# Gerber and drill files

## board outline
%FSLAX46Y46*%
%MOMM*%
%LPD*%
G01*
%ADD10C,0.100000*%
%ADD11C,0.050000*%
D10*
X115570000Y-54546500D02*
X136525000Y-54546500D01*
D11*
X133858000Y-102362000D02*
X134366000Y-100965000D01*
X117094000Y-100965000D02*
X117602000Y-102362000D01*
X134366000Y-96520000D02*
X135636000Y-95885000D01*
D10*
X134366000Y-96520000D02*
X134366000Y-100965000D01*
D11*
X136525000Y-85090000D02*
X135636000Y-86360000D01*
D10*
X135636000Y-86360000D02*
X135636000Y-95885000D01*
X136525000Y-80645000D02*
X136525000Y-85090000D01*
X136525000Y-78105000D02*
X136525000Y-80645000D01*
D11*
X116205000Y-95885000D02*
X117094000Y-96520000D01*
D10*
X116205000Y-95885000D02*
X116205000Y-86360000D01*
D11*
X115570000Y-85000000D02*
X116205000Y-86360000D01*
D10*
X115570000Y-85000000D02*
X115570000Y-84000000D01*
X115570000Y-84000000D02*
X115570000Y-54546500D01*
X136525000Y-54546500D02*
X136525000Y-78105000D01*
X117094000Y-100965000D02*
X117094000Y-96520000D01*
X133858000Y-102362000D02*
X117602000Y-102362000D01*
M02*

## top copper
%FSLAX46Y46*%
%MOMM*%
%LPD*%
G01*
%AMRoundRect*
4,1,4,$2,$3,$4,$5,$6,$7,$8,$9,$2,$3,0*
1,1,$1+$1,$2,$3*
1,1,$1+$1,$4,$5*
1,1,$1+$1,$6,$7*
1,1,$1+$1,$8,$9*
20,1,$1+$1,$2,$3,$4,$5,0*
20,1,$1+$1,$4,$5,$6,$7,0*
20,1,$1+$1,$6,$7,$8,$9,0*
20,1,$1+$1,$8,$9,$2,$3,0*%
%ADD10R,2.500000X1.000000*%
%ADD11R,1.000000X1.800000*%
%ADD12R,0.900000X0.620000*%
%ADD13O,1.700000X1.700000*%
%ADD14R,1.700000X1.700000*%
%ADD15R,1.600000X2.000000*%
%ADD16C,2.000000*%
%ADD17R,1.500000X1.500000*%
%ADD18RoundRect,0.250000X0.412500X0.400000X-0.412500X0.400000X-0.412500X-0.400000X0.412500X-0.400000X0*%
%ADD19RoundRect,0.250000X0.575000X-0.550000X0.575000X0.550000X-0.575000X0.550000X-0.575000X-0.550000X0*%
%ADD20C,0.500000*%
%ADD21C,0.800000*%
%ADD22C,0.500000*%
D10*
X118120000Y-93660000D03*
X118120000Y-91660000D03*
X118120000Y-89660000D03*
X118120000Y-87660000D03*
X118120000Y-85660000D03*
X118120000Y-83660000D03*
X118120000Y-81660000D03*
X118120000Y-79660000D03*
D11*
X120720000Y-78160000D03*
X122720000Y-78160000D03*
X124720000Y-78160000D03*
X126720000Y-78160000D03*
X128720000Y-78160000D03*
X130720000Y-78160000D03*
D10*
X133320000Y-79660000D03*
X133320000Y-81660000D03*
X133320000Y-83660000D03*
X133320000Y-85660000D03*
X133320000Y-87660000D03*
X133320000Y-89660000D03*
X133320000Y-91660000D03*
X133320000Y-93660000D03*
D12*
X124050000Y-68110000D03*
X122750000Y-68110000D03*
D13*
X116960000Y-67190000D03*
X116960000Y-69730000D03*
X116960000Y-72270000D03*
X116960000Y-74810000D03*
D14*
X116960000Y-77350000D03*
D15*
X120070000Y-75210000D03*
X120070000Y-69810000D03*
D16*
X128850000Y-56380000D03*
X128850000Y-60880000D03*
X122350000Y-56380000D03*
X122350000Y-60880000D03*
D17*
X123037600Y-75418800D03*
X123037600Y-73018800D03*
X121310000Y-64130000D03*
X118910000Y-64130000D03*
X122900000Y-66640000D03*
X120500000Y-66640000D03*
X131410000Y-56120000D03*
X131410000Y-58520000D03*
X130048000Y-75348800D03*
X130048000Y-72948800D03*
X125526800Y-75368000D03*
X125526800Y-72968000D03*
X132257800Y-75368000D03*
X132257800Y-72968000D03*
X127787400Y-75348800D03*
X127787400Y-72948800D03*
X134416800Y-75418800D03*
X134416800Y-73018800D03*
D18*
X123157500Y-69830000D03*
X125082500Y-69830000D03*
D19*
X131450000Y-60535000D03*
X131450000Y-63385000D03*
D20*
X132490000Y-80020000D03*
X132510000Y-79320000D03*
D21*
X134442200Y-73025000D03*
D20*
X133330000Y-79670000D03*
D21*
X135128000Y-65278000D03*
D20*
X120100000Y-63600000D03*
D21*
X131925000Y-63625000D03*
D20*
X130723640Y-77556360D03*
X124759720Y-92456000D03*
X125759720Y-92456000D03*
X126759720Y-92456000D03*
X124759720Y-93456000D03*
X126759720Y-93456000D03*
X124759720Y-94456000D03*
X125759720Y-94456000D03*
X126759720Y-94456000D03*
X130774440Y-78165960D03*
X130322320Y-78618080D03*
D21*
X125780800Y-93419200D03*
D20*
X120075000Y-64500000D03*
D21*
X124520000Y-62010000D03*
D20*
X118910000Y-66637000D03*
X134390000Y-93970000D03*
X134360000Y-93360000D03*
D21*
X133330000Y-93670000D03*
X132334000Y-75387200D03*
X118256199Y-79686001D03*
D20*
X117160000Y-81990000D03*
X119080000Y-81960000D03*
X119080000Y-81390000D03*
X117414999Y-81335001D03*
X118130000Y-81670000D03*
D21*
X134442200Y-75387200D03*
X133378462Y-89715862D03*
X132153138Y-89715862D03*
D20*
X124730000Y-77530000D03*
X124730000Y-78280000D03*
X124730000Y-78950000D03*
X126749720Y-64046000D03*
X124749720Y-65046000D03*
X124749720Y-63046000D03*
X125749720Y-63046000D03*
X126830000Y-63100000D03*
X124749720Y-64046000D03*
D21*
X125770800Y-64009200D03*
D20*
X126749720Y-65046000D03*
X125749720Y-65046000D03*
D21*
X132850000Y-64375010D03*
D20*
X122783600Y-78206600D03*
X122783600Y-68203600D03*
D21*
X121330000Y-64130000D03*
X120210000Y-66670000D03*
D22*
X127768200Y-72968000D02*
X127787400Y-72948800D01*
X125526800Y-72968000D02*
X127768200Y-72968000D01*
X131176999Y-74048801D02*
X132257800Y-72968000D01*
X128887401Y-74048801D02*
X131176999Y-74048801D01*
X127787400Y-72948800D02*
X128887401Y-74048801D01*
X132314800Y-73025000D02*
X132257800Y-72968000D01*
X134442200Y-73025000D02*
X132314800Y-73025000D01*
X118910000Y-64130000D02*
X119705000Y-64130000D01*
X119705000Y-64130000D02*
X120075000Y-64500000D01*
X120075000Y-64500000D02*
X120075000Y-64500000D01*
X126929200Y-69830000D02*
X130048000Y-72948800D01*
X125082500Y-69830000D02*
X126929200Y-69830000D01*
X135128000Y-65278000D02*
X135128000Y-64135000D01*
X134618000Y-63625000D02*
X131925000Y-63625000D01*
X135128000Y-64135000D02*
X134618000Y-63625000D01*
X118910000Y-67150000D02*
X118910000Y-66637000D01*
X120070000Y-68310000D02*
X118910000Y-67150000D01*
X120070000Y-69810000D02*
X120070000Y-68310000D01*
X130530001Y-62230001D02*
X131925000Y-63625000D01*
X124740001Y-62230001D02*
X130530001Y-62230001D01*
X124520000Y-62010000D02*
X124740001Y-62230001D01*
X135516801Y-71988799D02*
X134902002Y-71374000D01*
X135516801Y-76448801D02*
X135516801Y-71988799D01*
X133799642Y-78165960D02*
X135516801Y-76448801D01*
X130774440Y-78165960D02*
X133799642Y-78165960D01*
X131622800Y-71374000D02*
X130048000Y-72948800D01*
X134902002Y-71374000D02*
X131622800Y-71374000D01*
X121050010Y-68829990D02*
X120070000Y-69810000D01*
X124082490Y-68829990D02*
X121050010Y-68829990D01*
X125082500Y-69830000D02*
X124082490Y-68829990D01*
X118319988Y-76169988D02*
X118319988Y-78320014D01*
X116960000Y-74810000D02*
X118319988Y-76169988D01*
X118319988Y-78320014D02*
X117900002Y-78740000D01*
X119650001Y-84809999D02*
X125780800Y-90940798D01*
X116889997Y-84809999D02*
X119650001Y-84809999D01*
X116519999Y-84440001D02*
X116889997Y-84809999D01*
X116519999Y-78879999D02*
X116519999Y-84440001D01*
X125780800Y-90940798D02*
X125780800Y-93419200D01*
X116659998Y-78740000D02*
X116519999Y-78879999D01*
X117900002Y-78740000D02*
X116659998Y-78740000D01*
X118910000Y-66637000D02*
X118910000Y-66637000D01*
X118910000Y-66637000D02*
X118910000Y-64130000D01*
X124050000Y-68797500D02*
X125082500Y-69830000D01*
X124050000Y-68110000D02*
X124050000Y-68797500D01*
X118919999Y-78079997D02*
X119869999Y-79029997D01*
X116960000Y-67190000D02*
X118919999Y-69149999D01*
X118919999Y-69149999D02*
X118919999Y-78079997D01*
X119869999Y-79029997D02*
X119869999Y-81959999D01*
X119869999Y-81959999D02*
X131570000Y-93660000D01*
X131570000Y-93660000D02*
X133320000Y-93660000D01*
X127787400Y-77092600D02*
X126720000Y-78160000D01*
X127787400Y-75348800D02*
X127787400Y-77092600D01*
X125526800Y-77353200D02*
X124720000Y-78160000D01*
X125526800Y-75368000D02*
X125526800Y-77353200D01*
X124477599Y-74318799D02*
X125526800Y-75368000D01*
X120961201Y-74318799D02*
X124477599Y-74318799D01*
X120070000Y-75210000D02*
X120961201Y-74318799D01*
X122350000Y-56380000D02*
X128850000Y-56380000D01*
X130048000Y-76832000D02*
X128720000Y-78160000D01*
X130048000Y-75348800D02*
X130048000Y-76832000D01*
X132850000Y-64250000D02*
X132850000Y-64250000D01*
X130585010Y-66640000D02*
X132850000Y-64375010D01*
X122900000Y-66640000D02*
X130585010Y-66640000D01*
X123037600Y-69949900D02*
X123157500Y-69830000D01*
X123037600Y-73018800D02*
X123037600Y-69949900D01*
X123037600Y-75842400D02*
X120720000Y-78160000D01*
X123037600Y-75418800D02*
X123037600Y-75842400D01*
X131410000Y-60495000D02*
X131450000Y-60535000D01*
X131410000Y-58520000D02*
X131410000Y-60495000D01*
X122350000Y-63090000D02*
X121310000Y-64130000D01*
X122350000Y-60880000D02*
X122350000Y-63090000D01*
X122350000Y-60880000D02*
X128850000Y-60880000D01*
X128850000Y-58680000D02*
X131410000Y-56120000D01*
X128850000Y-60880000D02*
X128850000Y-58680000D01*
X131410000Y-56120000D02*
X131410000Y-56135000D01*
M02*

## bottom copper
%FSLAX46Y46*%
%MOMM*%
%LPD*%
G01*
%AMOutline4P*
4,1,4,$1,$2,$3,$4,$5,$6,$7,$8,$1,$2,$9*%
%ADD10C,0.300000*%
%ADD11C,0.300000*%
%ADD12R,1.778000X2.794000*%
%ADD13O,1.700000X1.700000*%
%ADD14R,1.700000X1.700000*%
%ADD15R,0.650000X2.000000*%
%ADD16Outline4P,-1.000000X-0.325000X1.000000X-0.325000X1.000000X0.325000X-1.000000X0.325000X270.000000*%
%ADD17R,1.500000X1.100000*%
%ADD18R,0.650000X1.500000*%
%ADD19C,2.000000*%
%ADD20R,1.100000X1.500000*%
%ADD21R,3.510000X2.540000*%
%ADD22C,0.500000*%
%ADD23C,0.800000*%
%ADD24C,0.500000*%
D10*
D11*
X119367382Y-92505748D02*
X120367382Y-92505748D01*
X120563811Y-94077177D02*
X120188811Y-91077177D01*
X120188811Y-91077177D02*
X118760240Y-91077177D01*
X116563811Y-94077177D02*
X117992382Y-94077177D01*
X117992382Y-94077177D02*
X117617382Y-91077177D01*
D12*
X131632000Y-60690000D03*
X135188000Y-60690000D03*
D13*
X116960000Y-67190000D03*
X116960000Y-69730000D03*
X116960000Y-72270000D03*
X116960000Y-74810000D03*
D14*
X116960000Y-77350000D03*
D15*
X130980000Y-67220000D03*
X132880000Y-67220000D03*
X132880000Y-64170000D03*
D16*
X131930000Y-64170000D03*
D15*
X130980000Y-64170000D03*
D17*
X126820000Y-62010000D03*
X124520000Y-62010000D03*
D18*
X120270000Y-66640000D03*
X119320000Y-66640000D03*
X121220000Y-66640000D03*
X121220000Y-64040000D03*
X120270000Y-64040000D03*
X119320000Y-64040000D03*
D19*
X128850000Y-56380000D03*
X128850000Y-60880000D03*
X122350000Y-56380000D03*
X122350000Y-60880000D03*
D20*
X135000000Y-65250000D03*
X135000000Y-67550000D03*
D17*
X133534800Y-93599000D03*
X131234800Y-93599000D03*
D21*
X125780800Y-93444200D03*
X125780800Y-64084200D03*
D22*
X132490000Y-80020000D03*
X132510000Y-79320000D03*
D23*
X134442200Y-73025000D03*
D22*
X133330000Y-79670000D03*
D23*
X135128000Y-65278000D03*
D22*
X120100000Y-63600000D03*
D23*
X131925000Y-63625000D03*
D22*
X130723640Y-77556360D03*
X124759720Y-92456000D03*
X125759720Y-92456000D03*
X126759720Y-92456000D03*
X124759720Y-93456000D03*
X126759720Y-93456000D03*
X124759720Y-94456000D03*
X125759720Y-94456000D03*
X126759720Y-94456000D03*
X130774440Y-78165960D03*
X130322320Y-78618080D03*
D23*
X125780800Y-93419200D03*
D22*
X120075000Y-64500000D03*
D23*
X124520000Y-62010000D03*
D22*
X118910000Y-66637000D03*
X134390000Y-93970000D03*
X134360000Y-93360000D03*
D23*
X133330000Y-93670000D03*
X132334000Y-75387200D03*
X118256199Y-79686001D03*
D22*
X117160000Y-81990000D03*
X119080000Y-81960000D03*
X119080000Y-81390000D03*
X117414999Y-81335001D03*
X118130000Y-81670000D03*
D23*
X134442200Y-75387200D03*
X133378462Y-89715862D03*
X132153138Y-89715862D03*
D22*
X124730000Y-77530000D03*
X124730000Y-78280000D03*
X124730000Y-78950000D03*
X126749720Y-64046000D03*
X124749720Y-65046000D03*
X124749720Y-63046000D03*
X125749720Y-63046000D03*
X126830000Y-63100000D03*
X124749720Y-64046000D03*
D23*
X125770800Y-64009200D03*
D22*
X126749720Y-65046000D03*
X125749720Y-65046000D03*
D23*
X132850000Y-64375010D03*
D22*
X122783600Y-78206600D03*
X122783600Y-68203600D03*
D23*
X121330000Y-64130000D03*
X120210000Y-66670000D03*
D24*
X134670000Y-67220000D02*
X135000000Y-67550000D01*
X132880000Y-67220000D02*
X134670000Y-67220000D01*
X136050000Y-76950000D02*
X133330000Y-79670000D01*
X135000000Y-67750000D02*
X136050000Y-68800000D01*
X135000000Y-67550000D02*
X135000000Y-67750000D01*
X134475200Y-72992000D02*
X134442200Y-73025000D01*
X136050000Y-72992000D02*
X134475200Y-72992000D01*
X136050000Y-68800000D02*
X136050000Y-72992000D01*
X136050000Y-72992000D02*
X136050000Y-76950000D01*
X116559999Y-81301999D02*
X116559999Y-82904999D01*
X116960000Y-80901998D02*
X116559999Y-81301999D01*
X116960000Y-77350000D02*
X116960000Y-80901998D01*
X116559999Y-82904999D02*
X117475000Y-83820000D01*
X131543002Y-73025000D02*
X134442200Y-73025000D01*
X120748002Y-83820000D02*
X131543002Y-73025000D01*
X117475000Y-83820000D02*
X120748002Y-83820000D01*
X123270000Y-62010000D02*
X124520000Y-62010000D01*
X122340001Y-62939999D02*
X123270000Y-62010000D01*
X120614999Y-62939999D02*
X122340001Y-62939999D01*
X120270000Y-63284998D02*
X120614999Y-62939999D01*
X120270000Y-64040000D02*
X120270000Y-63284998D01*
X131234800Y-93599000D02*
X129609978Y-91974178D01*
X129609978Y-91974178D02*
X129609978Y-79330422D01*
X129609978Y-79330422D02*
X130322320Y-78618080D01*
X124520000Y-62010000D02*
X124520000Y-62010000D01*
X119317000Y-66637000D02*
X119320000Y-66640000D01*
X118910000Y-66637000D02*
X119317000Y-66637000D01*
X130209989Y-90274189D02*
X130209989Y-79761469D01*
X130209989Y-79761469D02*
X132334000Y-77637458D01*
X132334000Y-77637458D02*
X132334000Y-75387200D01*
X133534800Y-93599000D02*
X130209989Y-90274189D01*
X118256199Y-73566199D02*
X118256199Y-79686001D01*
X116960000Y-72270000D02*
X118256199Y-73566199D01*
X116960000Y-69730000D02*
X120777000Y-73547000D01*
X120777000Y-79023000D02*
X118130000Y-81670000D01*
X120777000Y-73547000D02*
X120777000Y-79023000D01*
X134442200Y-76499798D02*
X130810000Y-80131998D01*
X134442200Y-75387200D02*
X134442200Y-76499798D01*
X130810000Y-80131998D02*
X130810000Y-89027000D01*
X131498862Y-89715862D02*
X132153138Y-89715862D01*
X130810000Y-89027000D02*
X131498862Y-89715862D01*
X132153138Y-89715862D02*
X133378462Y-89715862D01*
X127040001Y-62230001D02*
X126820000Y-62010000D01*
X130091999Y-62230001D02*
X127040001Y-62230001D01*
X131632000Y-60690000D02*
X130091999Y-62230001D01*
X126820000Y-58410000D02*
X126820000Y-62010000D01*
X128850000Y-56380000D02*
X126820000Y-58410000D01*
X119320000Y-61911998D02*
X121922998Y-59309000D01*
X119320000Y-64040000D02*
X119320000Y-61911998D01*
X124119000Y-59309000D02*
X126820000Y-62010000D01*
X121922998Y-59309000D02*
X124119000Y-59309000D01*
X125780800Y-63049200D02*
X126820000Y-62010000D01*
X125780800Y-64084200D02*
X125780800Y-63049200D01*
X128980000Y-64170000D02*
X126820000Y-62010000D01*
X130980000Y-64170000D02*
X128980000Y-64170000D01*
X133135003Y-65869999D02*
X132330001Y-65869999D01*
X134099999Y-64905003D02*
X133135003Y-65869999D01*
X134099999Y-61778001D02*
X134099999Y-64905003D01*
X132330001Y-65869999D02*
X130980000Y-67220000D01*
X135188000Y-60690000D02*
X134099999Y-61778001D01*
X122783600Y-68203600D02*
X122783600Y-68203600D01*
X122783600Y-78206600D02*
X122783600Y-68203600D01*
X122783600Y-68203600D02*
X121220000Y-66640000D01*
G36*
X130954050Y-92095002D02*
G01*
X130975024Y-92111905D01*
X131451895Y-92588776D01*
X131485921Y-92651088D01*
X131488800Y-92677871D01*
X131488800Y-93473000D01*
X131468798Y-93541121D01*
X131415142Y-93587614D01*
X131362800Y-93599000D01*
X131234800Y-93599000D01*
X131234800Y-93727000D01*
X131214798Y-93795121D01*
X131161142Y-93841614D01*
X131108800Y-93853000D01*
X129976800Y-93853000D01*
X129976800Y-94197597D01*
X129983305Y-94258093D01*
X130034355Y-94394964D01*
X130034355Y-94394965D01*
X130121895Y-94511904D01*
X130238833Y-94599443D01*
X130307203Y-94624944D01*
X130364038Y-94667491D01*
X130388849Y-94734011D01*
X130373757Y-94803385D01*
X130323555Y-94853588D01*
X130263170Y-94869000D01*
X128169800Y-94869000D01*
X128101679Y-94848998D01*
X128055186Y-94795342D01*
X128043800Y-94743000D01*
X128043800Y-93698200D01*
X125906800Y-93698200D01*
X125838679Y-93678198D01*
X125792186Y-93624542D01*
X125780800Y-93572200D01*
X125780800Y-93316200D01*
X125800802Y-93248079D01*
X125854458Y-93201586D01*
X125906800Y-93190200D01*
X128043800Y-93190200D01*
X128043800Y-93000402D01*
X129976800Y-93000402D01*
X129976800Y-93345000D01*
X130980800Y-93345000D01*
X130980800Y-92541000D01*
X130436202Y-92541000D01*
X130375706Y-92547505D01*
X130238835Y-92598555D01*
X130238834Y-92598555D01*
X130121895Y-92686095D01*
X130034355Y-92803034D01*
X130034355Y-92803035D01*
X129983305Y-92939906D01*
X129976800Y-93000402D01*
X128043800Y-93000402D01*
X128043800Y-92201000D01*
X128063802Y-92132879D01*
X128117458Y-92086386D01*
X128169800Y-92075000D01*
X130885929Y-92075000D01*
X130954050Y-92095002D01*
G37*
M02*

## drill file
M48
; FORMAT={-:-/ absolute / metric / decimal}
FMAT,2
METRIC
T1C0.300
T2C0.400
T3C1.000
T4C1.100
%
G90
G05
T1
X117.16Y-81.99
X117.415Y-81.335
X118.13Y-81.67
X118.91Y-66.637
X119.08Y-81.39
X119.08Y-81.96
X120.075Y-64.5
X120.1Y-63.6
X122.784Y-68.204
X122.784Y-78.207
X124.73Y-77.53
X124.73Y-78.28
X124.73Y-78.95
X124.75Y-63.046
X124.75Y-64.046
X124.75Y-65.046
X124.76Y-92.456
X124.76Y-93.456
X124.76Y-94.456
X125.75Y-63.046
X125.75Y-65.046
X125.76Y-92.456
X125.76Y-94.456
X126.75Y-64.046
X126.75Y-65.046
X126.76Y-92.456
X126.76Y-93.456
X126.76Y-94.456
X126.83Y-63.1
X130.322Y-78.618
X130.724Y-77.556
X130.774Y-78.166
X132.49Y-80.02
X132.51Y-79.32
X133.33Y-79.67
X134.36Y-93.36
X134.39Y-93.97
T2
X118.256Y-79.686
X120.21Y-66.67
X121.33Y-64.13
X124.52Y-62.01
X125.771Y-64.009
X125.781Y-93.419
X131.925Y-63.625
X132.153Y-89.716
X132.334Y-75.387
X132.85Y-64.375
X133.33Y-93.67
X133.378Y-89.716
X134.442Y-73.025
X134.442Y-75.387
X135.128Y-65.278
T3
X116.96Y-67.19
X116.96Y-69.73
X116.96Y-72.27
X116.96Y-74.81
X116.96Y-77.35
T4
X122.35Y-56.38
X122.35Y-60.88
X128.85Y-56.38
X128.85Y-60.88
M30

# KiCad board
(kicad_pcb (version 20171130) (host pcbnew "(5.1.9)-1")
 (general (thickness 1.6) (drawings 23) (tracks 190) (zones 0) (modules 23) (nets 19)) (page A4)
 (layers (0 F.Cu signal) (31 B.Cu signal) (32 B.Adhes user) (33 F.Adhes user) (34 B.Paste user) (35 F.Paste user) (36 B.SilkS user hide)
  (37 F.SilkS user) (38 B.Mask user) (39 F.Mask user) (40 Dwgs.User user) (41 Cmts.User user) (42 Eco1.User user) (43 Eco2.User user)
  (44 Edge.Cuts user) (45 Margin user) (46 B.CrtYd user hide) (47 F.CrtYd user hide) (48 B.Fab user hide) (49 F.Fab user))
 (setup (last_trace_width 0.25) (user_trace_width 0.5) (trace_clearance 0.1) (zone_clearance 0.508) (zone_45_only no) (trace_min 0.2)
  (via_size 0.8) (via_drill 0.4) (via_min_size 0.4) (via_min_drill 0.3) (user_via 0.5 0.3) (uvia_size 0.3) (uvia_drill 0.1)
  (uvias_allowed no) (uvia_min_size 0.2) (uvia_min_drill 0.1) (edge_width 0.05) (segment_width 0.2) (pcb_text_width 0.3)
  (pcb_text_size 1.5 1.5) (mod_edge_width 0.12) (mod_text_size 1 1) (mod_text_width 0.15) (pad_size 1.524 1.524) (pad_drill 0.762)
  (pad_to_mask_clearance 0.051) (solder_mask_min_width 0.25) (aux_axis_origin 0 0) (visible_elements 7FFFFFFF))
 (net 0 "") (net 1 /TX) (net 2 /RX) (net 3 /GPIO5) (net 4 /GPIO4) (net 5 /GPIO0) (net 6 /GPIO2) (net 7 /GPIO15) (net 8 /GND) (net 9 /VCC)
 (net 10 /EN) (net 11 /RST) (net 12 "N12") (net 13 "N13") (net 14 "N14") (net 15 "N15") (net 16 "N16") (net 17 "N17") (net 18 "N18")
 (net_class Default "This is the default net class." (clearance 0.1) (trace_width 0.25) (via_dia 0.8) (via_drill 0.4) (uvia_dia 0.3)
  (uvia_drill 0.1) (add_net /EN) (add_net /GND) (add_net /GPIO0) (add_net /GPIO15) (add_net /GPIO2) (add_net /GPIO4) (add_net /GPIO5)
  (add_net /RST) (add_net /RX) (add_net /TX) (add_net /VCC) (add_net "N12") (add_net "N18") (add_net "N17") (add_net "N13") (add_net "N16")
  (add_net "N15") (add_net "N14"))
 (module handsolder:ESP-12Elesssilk (layer F.Cu) (at 125.72 90.16 180)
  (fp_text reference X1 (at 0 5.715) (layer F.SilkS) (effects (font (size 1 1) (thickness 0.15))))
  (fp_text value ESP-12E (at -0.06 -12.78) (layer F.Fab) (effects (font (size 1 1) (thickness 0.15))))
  (pad 22 smd rect (at 7.6 -3.5 180) (size 2.5 1) (layers F.Cu F.Paste F.Mask))
  (pad 21 smd rect (at 7.6 -1.5 180) (size 2.5 1) (layers F.Cu F.Paste F.Mask))
  (pad 20 smd rect (at 7.6 0.5 180) (size 2.5 1) (layers F.Cu F.Paste F.Mask))
  (pad 19 smd rect (at 7.6 2.5 180) (size 2.5 1) (layers F.Cu F.Paste F.Mask))
  (pad 18 smd rect (at 7.6 4.5 180) (size 2.5 1) (layers F.Cu F.Paste F.Mask))
  (pad 17 smd rect (at 7.6 6.5 180) (size 2.5 1) (layers F.Cu F.Paste F.Mask))
  (pad 16 smd rect (at 7.6 8.5 180) (size 2.5 1) (layers F.Cu F.Paste F.Mask) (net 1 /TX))
  (pad 15 smd rect (at 7.6 10.5 180) (size 2.5 1) (layers F.Cu F.Paste F.Mask) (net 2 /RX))
  (pad 14 smd rect (at 5 12 180) (size 1 1.8) (layers F.Cu F.Paste F.Mask) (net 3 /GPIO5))
  (pad 13 smd rect (at 3 12 180) (size 1 1.8) (layers F.Cu F.Paste F.Mask) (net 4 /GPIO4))
  (pad 12 smd rect (at 1 12 180) (size 1 1.8) (layers F.Cu F.Paste F.Mask) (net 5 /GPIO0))
  (pad 11 smd rect (at -1 12 180) (size 1 1.8) (layers F.Cu F.Paste F.Mask) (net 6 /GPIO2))
  (pad 10 smd rect (at -3 12 180) (size 1 1.8) (layers F.Cu F.Paste F.Mask) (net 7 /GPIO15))
  (pad 9 smd rect (at -5 12 180) (size 1 1.8) (layers F.Cu F.Paste F.Mask) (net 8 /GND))
  (pad 8 smd rect (at -7.6 10.5 180) (size 2.5 1) (layers F.Cu F.Paste F.Mask) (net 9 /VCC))
  (pad 7 smd rect (at -7.6 8.5 180) (size 2.5 1) (layers F.Cu F.Paste F.Mask))
  (pad 6 smd rect (at -7.6 6.5 180) (size 2.5 1) (layers F.Cu F.Paste F.Mask))
  (pad 5 smd rect (at -7.6 4.5 180) (size 2.5 1) (layers F.Cu F.Paste F.Mask))
  (pad 4 smd rect (at -7.6 2.5 180) (size 2.5 1) (layers F.Cu F.Paste F.Mask))
  (pad 3 smd rect (at -7.6 0.5 180) (size 2.5 1) (layers F.Cu F.Paste F.Mask) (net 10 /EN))
  (pad 2 smd rect (at -7.6 -1.5 180) (size 2.5 1) (layers F.Cu F.Paste F.Mask))
  (pad 1 smd rect (at -7.6 -3.5 180) (size 2.5 1) (layers F.Cu F.Paste F.Mask) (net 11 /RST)))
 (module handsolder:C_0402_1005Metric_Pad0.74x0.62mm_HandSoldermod (layer F.Cu) (at 123.4 68.11)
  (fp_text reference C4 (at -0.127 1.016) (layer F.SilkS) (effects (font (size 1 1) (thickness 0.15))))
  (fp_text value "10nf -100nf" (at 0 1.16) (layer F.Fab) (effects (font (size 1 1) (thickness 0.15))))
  (pad 2 smd rect (at 0.65 0) (size 0.9 0.62) (layers F.Cu F.Paste F.Mask) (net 8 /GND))
  (pad 1 smd rect (at -0.65 0) (size 0.9 0.62) (layers F.Cu F.Paste F.Mask) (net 4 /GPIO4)))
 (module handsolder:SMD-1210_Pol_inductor (layer B.Cu) (at 133.41 60.69)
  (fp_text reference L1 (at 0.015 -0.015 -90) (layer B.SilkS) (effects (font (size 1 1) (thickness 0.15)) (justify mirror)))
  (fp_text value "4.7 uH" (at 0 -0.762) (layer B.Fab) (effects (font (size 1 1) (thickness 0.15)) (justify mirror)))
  (pad 1 smd rect (at -1.778 0) (size 1.778 2.794) (layers B.Cu B.Paste B.Mask) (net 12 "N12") (zone_connect 2))
  (pad 2 smd rect (at 1.778 0) (size 1.778 2.794) (layers B.Cu B.Paste B.Mask) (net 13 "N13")))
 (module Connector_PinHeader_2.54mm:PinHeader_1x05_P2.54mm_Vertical (layer F.Cu) (at 116.96 77.35 180)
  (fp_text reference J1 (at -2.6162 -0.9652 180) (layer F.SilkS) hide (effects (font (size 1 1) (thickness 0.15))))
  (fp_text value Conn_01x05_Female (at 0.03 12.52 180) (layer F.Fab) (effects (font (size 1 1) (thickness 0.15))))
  (pad 5 thru_hole oval (at 0 10.16 180) (size 1.7 1.7) (drill 1) (layers *.Cu *.Mask) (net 11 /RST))
  (pad 4 thru_hole oval (at 0 7.62 180) (size 1.7 1.7) (drill 1) (layers *.Cu *.Mask) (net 1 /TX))
  (pad 3 thru_hole oval (at 0 5.08 180) (size 1.7 1.7) (drill 1) (layers *.Cu *.Mask) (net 2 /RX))
  (pad 2 thru_hole oval (at 0 2.54 180) (size 1.7 1.7) (drill 1) (layers *.Cu *.Mask) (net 8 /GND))
  (pad 1 thru_hole rect (at 0 0 180) (size 1.7 1.7) (drill 1) (layers *.Cu *.Mask) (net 9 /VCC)))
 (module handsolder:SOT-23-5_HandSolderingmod (layer B.Cu) (at 131.93 65.72 270)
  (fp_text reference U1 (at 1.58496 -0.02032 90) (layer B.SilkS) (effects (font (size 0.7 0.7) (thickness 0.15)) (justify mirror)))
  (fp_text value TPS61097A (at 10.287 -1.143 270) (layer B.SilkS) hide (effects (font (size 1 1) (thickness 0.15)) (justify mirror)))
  (pad 5 smd rect (at 1.5 0.95 270) (size 2 0.65) (layers B.Cu B.Paste B.Mask) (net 13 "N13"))
  (pad 4 smd rect (at 1.5 -0.95 270) (size 2 0.65) (layers B.Cu B.Paste B.Mask) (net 9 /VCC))
  (pad 3 smd rect (at -1.55 -0.95 270) (size 2 0.65) (layers B.Cu B.Paste B.Mask) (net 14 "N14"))
  (pad 2 smd trapezoid (at -1.55 0 270) (size 2 0.65) (layers B.Cu B.Paste B.Mask) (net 8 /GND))
  (pad 1 smd rect (at -1.55 0.95 270) (size 2 0.65) (layers B.Cu B.Paste B.Mask) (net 12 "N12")))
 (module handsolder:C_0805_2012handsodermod (layer B.Cu) (at 125.67 62.01)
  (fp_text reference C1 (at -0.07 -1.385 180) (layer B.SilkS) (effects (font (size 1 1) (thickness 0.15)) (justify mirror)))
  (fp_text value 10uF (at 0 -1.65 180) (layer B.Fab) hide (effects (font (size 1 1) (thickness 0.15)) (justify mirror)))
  (pad 2 smd rect (at 1.15 0) (size 1.5 1.1) (layers B.Cu B.Paste B.Mask) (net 12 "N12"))
  (pad 1 smd rect (at -1.15 0) (size 1.5 1.1) (layers B.Cu B.Paste B.Mask) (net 8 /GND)))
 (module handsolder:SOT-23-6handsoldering (layer B.Cu) (at 120.27 65.34 270)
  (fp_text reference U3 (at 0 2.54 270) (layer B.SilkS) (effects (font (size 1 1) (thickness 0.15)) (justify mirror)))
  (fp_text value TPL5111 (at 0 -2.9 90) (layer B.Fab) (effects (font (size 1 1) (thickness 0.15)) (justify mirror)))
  (pad 5 smd rect (at 1.3 0 270) (size 1.5 0.65) (layers B.Cu B.Paste B.Mask) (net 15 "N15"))
  (pad 6 smd rect (at 1.3 0.95 270) (size 1.5 0.65) (layers B.Cu B.Paste B.Mask) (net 8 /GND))
  (pad 4 smd rect (at 1.3 -0.95 270) (size 1.5 0.65) (layers B.Cu B.Paste B.Mask) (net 4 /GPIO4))
  (pad 3 smd rect (at -1.3 -0.95 270) (size 1.5 0.65) (layers B.Cu B.Paste B.Mask) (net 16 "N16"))
  (pad 2 smd rect (at -1.3 0 270) (size 1.5 0.65) (layers B.Cu B.Paste B.Mask) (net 8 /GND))
  (pad 1 smd rect (at -1.3 0.95 270) (size 1.5 0.65) (layers B.Cu B.Paste B.Mask) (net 12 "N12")))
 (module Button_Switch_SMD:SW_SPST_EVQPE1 (layer F.Cu) (at 120.07 72.51 90)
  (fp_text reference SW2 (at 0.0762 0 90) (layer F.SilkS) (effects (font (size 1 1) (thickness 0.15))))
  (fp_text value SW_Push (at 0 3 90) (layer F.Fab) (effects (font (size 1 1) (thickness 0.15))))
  (pad 1 smd rect (at -2.7 0 90) (size 2 1.6) (layers F.Cu F.Paste F.Mask) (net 5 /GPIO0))
  (pad 2 smd rect (at 2.7 0 90) (size 2 1.6) (layers F.Cu F.Paste F.Mask) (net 8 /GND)))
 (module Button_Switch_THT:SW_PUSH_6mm (layer F.Cu) (at 122.35 56.38)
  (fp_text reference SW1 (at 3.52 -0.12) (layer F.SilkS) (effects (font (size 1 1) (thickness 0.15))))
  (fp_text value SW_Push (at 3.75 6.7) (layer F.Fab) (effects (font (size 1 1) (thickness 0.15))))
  (pad 1 thru_hole circle (at 6.5 0 90) (size 2 2) (drill 1.1) (layers *.Cu *.Mask) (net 12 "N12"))
  (pad 2 thru_hole circle (at 6.5 4.5 90) (size 2 2) (drill 1.1) (layers *.Cu *.Mask) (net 16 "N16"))
  (pad 1 thru_hole circle (at 0 0 90) (size 2 2) (drill 1.1) (layers *.Cu *.Mask) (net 12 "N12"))
  (pad 2 thru_hole circle (at 0 4.5 90) (size 2 2) (drill 1.1) (layers *.Cu *.Mask) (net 16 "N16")))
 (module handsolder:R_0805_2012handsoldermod (layer F.Cu) (at 123.0376 74.2188 270)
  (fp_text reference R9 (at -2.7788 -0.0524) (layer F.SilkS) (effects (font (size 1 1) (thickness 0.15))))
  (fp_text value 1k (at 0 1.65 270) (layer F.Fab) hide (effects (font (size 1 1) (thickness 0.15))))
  (pad 2 smd rect (at 1.2 0 270) (size 1.5 1.5) (layers F.Cu F.Paste F.Mask) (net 3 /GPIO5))
  (pad 1 smd rect (at -1.2 0 270) (size 1.5 1.5) (layers F.Cu F.Paste F.Mask) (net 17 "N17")))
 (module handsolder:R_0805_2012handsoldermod (layer F.Cu) (at 120.11 64.13)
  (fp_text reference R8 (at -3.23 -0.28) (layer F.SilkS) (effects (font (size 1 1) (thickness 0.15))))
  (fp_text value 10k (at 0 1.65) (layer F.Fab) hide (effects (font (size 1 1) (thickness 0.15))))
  (pad 2 smd rect (at 1.2 0) (size 1.5 1.5) (layers F.Cu F.Paste F.Mask) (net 16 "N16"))
  (pad 1 smd rect (at -1.2 0) (size 1.5 1.5) (layers F.Cu F.Paste F.Mask) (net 8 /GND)))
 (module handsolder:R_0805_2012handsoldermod (layer F.Cu) (at 121.7 66.64)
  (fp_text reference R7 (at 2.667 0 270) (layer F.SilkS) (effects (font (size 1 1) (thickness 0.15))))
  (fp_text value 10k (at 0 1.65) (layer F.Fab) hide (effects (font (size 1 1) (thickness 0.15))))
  (pad 2 smd rect (at 1.2 0) (size 1.5 1.5) (layers F.Cu F.Paste F.Mask) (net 14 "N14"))
  (pad 1 smd rect (at -1.2 0) (size 1.5 1.5) (layers F.Cu F.Paste F.Mask) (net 15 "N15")))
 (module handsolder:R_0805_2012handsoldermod (layer F.Cu) (at 131.41 57.32 90)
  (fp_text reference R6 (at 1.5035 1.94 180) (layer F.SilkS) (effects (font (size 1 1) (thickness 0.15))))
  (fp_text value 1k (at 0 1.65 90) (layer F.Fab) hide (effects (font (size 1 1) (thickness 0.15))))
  (pad 2 smd rect (at 1.2 0 90) (size 1.5 1.5) (layers F.Cu F.Paste F.Mask) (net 16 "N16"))
  (pad 1 smd rect (at -1.2 0 90) (size 1.5 1.5) (layers F.Cu F.Paste F.Mask) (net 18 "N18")))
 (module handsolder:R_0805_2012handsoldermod (layer F.Cu) (at 130.048 74.1488 270)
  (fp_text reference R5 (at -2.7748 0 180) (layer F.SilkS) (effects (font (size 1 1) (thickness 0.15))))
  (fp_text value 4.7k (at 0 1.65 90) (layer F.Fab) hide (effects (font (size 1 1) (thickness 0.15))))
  (pad 2 smd rect (at 1.2 0 270) (size 1.5 1.5) (layers F.Cu F.Paste F.Mask) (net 7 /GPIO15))
  (pad 1 smd rect (at -1.2 0 270) (size 1.5 1.5) (layers F.Cu F.Paste F.Mask) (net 8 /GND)))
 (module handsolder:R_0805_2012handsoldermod (layer F.Cu) (at 125.5268 74.168 270)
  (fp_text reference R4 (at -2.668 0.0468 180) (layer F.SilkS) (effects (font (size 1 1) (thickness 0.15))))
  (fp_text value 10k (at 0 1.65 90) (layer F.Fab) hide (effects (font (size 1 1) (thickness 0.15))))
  (pad 2 smd rect (at 1.2 0 270) (size 1.5 1.5) (layers F.Cu F.Paste F.Mask) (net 5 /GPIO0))
  (pad 1 smd rect (at -1.2 0 270) (size 1.5 1.5) (layers F.Cu F.Paste F.Mask) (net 9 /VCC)))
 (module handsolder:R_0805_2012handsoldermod (layer F.Cu) (at 132.2578 74.168 270)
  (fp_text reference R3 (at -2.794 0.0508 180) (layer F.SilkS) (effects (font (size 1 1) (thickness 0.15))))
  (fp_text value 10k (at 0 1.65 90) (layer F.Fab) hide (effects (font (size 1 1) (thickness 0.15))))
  (pad 2 smd rect (at 1.2 0 270) (size 1.5 1.5) (layers F.Cu F.Paste F.Mask) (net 11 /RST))
  (pad 1 smd rect (at -1.2 0 270) (size 1.5 1.5) (layers F.Cu F.Paste F.Mask) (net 9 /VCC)))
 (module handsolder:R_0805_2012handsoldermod (layer F.Cu) (at 127.7874 74.1488 270)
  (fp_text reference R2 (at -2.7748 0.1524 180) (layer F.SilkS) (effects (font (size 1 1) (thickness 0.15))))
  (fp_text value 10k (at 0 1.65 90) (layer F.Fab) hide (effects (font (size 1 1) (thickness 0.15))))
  (pad 2 smd rect (at 1.2 0 270) (size 1.5 1.5) (layers F.Cu F.Paste F.Mask) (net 6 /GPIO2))
  (pad 1 smd rect (at -1.2 0 270) (size 1.5 1.5) (layers F.Cu F.Paste F.Mask) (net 9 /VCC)))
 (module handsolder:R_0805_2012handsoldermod (layer F.Cu) (at 134.4168 74.2188 270)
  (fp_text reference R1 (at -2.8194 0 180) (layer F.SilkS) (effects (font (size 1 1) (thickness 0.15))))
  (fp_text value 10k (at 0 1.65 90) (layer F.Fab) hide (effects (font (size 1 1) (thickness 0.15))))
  (pad 2 smd rect (at 1.2 0 270) (size 1.5 1.5) (layers F.Cu F.Paste F.Mask) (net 10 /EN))
  (pad 1 smd rect (at -1.2 0 270) (size 1.5 1.5) (layers F.Cu F.Paste F.Mask) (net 9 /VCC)))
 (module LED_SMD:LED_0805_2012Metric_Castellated (layer F.Cu) (at 124.12 69.83 180)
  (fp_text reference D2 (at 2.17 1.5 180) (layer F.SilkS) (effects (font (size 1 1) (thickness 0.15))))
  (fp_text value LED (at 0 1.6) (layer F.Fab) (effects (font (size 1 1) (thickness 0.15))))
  (pad 2 smd roundrect (at 0.9625 0 180) (size 1.325 1.3) (layers F.Cu F.Paste F.Mask) (roundrect_rratio 0.1923076923076923) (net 17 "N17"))
  (pad 1 smd roundrect (at -0.9625 0 180) (size 1.325 1.3) (layers F.Cu F.Paste F.Mask) (roundrect_rratio 0.1923076923076923) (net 8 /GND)))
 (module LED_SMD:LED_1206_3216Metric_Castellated (layer F.Cu) (at 131.45 61.96 90)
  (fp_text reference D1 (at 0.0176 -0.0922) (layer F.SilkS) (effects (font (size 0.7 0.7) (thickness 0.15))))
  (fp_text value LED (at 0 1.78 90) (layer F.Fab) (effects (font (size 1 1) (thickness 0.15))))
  (pad 2 smd roundrect (at 1.425 0 90) (size 1.6 1.65) (layers F.Cu F.Paste F.Mask) (roundrect_rratio 0.15625) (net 18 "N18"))
  (pad 1 smd roundrect (at -1.425 0 90) (size 1.6 1.65) (layers F.Cu F.Paste F.Mask) (roundrect_rratio 0.15625) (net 8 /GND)))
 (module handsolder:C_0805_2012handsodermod (layer B.Cu) (at 135 66.4 90)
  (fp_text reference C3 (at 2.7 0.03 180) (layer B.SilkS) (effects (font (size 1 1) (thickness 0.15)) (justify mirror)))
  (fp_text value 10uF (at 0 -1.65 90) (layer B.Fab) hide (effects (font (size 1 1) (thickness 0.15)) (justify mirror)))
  (pad 2 smd rect (at 1.15 0 90) (size 1.5 1.1) (layers B.Cu B.Paste B.Mask) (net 8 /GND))
  (pad 1 smd rect (at -1.15 0 90) (size 1.5 1.1) (layers B.Cu B.Paste B.Mask) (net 9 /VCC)))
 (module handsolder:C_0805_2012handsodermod (layer B.Cu) (at 132.3848 93.599)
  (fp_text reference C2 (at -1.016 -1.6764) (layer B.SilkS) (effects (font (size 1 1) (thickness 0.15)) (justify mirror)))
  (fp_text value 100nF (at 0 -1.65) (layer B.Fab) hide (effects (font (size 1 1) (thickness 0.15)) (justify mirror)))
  (pad 2 smd rect (at 1.15 0) (size 1.5 1.1) (layers B.Cu B.Paste B.Mask) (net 11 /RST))
  (pad 1 smd rect (at -1.15 0) (size 1.5 1.1) (layers B.Cu B.Paste B.Mask) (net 8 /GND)))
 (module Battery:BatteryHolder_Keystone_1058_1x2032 (layer B.Cu) (at 125.7808 78.7642 270)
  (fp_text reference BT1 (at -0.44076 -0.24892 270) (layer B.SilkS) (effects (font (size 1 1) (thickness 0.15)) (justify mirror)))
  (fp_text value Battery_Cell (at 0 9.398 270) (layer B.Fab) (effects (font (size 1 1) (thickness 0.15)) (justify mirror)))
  (pad 2 smd rect (at 14.68 0 270) (size 2.54 3.51) (layers B.Cu B.Paste B.Mask) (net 8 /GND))
  (pad 1 smd rect (at -14.68 0 270) (size 2.54 3.51) (layers B.Cu B.Paste B.Mask) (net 12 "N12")))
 (gr_line (start 115.57 54.5465) (end 136.525 54.5465) (layer Edge.Cuts) (width 0.1))
 (gr_line (start 133.858 102.362) (end 134.366 100.965) (layer Edge.Cuts) (width 0.05))
 (gr_line (start 117.094 100.965) (end 117.602 102.362) (layer Edge.Cuts) (width 0.05))
 (gr_line (start 134.366 96.52) (end 135.636 95.885) (layer Edge.Cuts) (width 0.05))
 (gr_line (start 134.366 96.52) (end 134.366 100.965) (layer Edge.Cuts) (width 0.1))
 (gr_line (start 136.525 85.09) (end 135.636 86.36) (layer Edge.Cuts) (width 0.05))
 (gr_line (start 135.636 86.36) (end 135.636 95.885) (layer Edge.Cuts) (width 0.1))
 (gr_line (start 136.525 80.645) (end 136.525 85.09) (layer Edge.Cuts) (width 0.1))
 (gr_line (start 136.525 78.105) (end 136.525 80.645) (layer Edge.Cuts) (width 0.1))
 (gr_line (start 116.205 95.885) (end 117.094 96.52) (layer Edge.Cuts) (width 0.05))
 (gr_line (start 116.205 95.885) (end 116.205 86.36) (layer Edge.Cuts) (width 0.1))
 (gr_line (start 115.57 85) (end 116.205 86.36) (layer Edge.Cuts) (width 0.05))
 (gr_line (start 115.57 85) (end 115.57 84) (layer Edge.Cuts) (width 0.1))
 (gr_line (start 115.57 84) (end 115.57 54.5465) (layer Edge.Cuts) (width 0.1))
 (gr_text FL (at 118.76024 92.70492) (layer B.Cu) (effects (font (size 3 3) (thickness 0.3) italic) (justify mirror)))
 (gr_line (start 136.525 54.5465) (end 136.525 78.105) (layer Edge.Cuts) (width 0.1))
 (gr_line (start 117.094 100.965) (end 117.094 96.52) (layer Edge.Cuts) (width 0.1))
 (gr_line (start 133.858 102.362) (end 117.602 102.362) (layer Edge.Cuts) (width 0.1))
 (via (at 132.49 80.02) (size 0.5) (drill 0.3) (layers F.Cu B.Cu) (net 9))
 (via (at 132.51 79.32) (size 0.5) (drill 0.3) (layers F.Cu B.Cu) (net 9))
 (via (at 134.4422 73.025) (size 0.8) (drill 0.4) (layers F.Cu B.Cu) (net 9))
 (via (at 133.33 79.67) (size 0.5) (drill 0.3) (layers F.Cu B.Cu) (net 9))
 (segment (start 127.7682 72.968) (end 127.7874 72.9488) (width 0.5) (layer F.Cu) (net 9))
 (segment (start 125.5268 72.968) (end 127.7682 72.968) (width 0.5) (layer F.Cu) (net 9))
 (segment (start 131.176999 74.048801) (end 132.2578 72.968) (width 0.5) (layer F.Cu) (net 9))
 (segment (start 128.887401 74.048801) (end 131.176999 74.048801) (width 0.5) (layer F.Cu) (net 9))
 (segment (start 127.7874 72.9488) (end 128.887401 74.048801) (width 0.5) (layer F.Cu) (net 9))
 (segment (start 134.67 67.22) (end 135 67.55) (width 0.5) (layer B.Cu) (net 9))
 (segment (start 132.88 67.22) (end 134.67 67.22) (width 0.5) (layer B.Cu) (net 9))
 (segment (start 136.05 76.95) (end 133.33 79.67) (width 0.5) (layer B.Cu) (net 9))
 (segment (start 135 67.75) (end 136.05 68.8) (width 0.5) (layer B.Cu) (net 9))
 (segment (start 135 67.55) (end 135 67.75) (width 0.5) (layer B.Cu) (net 9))
 (segment (start 134.4752 72.992) (end 134.4422 73.025) (width 0.5) (layer B.Cu) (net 9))
 (segment (start 136.05 72.992) (end 134.4752 72.992) (width 0.5) (layer B.Cu) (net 9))
 (segment (start 136.05 68.8) (end 136.05 72.992) (width 0.5) (layer B.Cu) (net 9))
 (segment (start 136.05 72.992) (end 136.05 76.95) (width 0.5) (layer B.Cu) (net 9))
 (segment (start 132.3148 73.025) (end 132.2578 72.968) (width 0.5) (layer F.Cu) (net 9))
 (segment (start 134.4422 73.025) (end 132.3148 73.025) (width 0.5) (layer F.Cu) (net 9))
 (segment (start 116.559999 81.301999) (end 116.559999 82.904999) (width 0.5) (layer B.Cu) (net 9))
 (segment (start 116.96 80.901998) (end 116.559999 81.301999) (width 0.5) (layer B.Cu) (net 9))
 (segment (start 116.96 77.35) (end 116.96 80.901998) (width 0.5) (layer B.Cu) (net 9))
 (segment (start 116.559999 82.904999) (end 117.475 83.82) (width 0.5) (layer B.Cu) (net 9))
 (segment (start 131.543002 73.025) (end 134.4422 73.025) (width 0.5) (layer B.Cu) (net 9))
 (segment (start 120.748002 83.82) (end 131.543002 73.025) (width 0.5) (layer B.Cu) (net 9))
 (segment (start 117.475 83.82) (end 120.748002 83.82) (width 0.5) (layer B.Cu) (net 9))
 (via (at 135.128 65.278) (size 0.8) (drill 0.4) (layers F.Cu B.Cu) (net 8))
 (via (at 120.1 63.6) (size 0.5) (drill 0.3) (layers F.Cu B.Cu) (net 8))
 (via (at 131.925 63.625) (size 0.8) (drill 0.4) (layers F.Cu B.Cu) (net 8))
 (via (at 130.72364 77.55636) (size 0.5) (drill 0.3) (layers F.Cu B.Cu) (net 8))
 (via (at 124.75972 92.456) (size 0.5) (drill 0.3) (layers F.Cu B.Cu) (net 8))
 (via (at 125.75972 92.456) (size 0.5) (drill 0.3) (layers F.Cu B.Cu) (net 8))
 (via (at 126.75972 92.456) (size 0.5) (drill 0.3) (layers F.Cu B.Cu) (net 8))
 (via (at 124.75972 93.456) (size 0.5) (drill 0.3) (layers F.Cu B.Cu) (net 8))
 (via (at 126.75972 93.456) (size 0.5) (drill 0.3) (layers F.Cu B.Cu) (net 8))
 (via (at 124.75972 94.456) (size 0.5) (drill 0.3) (layers F.Cu B.Cu) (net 8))
 (via (at 125.75972 94.456) (size 0.5) (drill 0.3) (layers F.Cu B.Cu) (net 8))
 (via (at 126.75972 94.456) (size 0.5) (drill 0.3) (layers F.Cu B.Cu) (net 8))
 (via (at 130.77444 78.16596) (size 0.5) (drill 0.3) (layers F.Cu B.Cu) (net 8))
 (via (at 130.32232 78.61808) (size 0.5) (drill 0.3) (layers F.Cu B.Cu) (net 8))
 (via (at 125.7808 93.4192) (size 0.8) (drill 0.4) (layers F.Cu B.Cu) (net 8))
 (segment (start 118.91 64.13) (end 119.705 64.13) (width 0.5) (layer F.Cu) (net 8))
 (segment (start 119.705 64.13) (end 120.075 64.5) (width 0.5) (layer F.Cu) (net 8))
 (segment (start 120.075 64.5) (end 120.075 64.5) (width 0.5) (layer F.Cu) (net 8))
 (via (at 120.075 64.5) (size 0.5) (drill 0.3) (layers F.Cu B.Cu) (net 8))
 (segment (start 126.9292 69.83) (end 130.048 72.9488) (width 0.5) (layer F.Cu) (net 8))
 (segment (start 125.0825 69.83) (end 126.9292 69.83) (width 0.5) (layer F.Cu) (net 8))
 (segment (start 123.27 62.01) (end 124.52 62.01) (width 0.5) (layer B.Cu) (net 8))
 (segment (start 122.340001 62.939999) (end 123.27 62.01) (width 0.5) (layer B.Cu) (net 8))
 (segment (start 120.614999 62.939999) (end 122.340001 62.939999) (width 0.5) (layer B.Cu) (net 8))
 (segment (start 120.27 63.284998) (end 120.614999 62.939999) (width 0.5) (layer B.Cu) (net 8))
 (segment (start 120.27 64.04) (end 120.27 63.284998) (width 0.5) (layer B.Cu) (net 8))
 (segment (start 135.128 65.278) (end 135.128 64.135) (width 0.5) (layer F.Cu) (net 8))
 (segment (start 134.618 63.625) (end 131.925 63.625) (width 0.5) (layer F.Cu) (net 8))
 (segment (start 135.128 64.135) (end 134.618 63.625) (width 0.5) (layer F.Cu) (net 8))
 (segment (start 118.91 67.15) (end 118.91 66.637) (width 0.5) (layer F.Cu) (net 8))
 (segment (start 120.07 68.31) (end 118.91 67.15) (width 0.5) (layer F.Cu) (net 8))
 (segment (start 120.07 69.81) (end 120.07 68.31) (width 0.5) (layer F.Cu) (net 8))
 (segment (start 131.2348 93.599) (end 129.609978 91.974178) (width 0.5) (layer B.Cu) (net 8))
 (segment (start 129.609978 91.974178) (end 129.609978 79.330422) (width 0.5) (layer B.Cu) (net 8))
 (segment (start 129.609978 79.330422) (end 130.32232 78.61808) (width 0.5) (layer B.Cu) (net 8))
 (segment (start 124.52 62.01) (end 124.52 62.01) (width 0.5) (layer B.Cu) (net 8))
 (via (at 124.52 62.01) (size 0.8) (drill 0.4) (layers F.Cu B.Cu) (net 8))
 (segment (start 130.530001 62.230001) (end 131.925 63.625) (width 0.5) (layer F.Cu) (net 8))
 (segment (start 124.740001 62.230001) (end 130.530001 62.230001) (width 0.5) (layer F.Cu) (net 8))
 (segment (start 124.52 62.01) (end 124.740001 62.230001) (width 0.5) (layer F.Cu) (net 8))
 (segment (start 135.516801 71.988799) (end 134.902002 71.374) (width 0.5) (layer F.Cu) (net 8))
 (segment (start 135.516801 76.448801) (end 135.516801 71.988799) (width 0.5) (layer F.Cu) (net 8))
 (segment (start 133.799642 78.16596) (end 135.516801 76.448801) (width 0.5) (layer F.Cu) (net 8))
 (segment (start 130.77444 78.16596) (end 133.799642 78.16596) (width 0.5) (layer F.Cu) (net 8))
 (segment (start 131.6228 71.374) (end 130.048 72.9488) (width 0.5) (layer F.Cu) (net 8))
 (segment (start 134.902002 71.374) (end 131.6228 71.374) (width 0.5) (layer F.Cu) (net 8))
 (segment (start 121.05001 68.82999) (end 120.07 69.81) (width 0.5) (layer F.Cu) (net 8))
 (segment (start 124.08249 68.82999) (end 121.05001 68.82999) (width 0.5) (layer F.Cu) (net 8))
 (segment (start 125.0825 69.83) (end 124.08249 68.82999) (width 0.5) (layer F.Cu) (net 8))
 (segment (start 118.319988 76.169988) (end 118.319988 78.320014) (width 0.5) (layer F.Cu) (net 8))
 (segment (start 116.96 74.81) (end 118.319988 76.169988) (width 0.5) (layer F.Cu) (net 8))
 (segment (start 118.319988 78.320014) (end 117.900002 78.74) (width 0.5) (layer F.Cu) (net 8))
 (segment (start 119.650001 84.809999) (end 125.7808 90.940798) (width 0.5) (layer F.Cu) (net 8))
 (segment (start 116.889997 84.809999) (end 119.650001 84.809999) (width 0.5) (layer F.Cu) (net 8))
 (segment (start 116.519999 84.440001) (end 116.889997 84.809999) (width 0.5) (layer F.Cu) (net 8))
 (segment (start 116.519999 78.879999) (end 116.519999 84.440001) (width 0.5) (layer F.Cu) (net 8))
 (segment (start 125.7808 90.940798) (end 125.7808 93.4192) (width 0.5) (layer F.Cu) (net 8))
 (segment (start 116.659998 78.74) (end 116.519999 78.879999) (width 0.5) (layer F.Cu) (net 8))
 (segment (start 117.900002 78.74) (end 116.659998 78.74) (width 0.5) (layer F.Cu) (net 8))
 (segment (start 118.91 66.637) (end 118.91 66.637) (width 0.5) (layer F.Cu) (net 8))
 (segment (start 118.91 66.637) (end 118.91 64.13) (width 0.5) (layer F.Cu) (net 8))
 (via (at 118.91 66.637) (size 0.5) (drill 0.3) (layers F.Cu B.Cu) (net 8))
 (segment (start 119.317 66.637) (end 119.32 66.64) (width 0.5) (layer B.Cu) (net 8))
 (segment (start 118.91 66.637) (end 119.317 66.637) (width 0.5) (layer B.Cu) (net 8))
 (segment (start 124.05 68.7975) (end 125.0825 69.83) (width 0.5) (layer F.Cu) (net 8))
 (segment (start 124.05 68.11) (end 124.05 68.7975) (width 0.5) (layer F.Cu) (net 8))
 (via (at 134.39 93.97) (size 0.5) (drill 0.3) (layers F.Cu B.Cu) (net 11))
 (via (at 134.36 93.36) (size 0.5) (drill 0.3) (layers F.Cu B.Cu) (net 11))
 (via (at 133.33 93.67) (size 0.8) (drill 0.4) (layers F.Cu B.Cu) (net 11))
 (via (at 132.334 75.3872) (size 0.8) (drill 0.4) (layers F.Cu B.Cu) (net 11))
 (segment (start 130.209989 90.274189) (end 130.209989 79.761469) (width 0.5) (layer B.Cu) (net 11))
 (segment (start 130.209989 79.761469) (end 132.334 77.637458) (width 0.5) (layer B.Cu) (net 11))
 (segment (start 132.334 77.637458) (end 132.334 75.3872) (width 0.5) (layer B.Cu) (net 11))
 (segment (start 133.5348 93.599) (end 130.209989 90.274189) (width 0.5) (layer B.Cu) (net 11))
 (segment (start 118.919999 78.079997) (end 119.869999 79.029997) (width 0.5) (layer F.Cu) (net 11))
 (segment (start 116.96 67.19) (end 118.919999 69.149999) (width 0.5) (layer F.Cu) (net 11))
 (segment (start 118.919999 69.149999) (end 118.919999 78.079997) (width 0.5) (layer F.Cu) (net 11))
 (segment (start 119.869999 79.029997) (end 119.869999 81.959999) (width 0.5) (layer F.Cu) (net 11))
 (segment (start 119.869999 81.959999) (end 131.57 93.66) (width 0.5) (layer F.Cu) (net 11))
 (segment (start 131.57 93.66) (end 133.32 93.66) (width 0.5) (layer F.Cu) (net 11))
 (via (at 118.256199 79.686001) (size 0.8) (drill 0.4) (layers F.Cu B.Cu) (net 2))
 (segment (start 118.256199 73.566199) (end 118.256199 79.686001) (width 0.5) (layer B.Cu) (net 2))
 (segment (start 116.96 72.27) (end 118.256199 73.566199) (width 0.5) (layer B.Cu) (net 2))
 (via (at 117.16 81.99) (size 0.5) (drill 0.3) (layers F.Cu B.Cu) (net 1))
 (via (at 119.08 81.96) (size 0.5) (drill 0.3) (layers F.Cu B.Cu) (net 1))
 (via (at 119.08 81.39) (size 0.5) (drill 0.3) (layers F.Cu B.Cu) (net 1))
 (via (at 117.414999 81.335001) (size 0.5) (drill 0.3) (layers F.Cu B.Cu) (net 1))
 (via (at 118.13 81.67) (size 0.5) (drill 0.3) (layers F.Cu B.Cu) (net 1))
 (segment (start 116.96 69.73) (end 120.777 73.547) (width 0.5) (layer B.Cu) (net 1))
 (segment (start 120.777 79.023) (end 118.13 81.67) (width 0.5) (layer B.Cu) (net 1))
 (segment (start 120.777 73.547) (end 120.777 79.023) (width 0.5) (layer B.Cu) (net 1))
 (via (at 134.4422 75.3872) (size 0.8) (drill 0.4) (layers F.Cu B.Cu) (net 10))
 (via (at 133.378462 89.715862) (size 0.8) (drill 0.4) (layers F.Cu B.Cu) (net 10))
 (segment (start 134.4422 76.499798) (end 130.81 80.131998) (width 0.5) (layer B.Cu) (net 10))
 (segment (start 134.4422 75.3872) (end 134.4422 76.499798) (width 0.5) (layer B.Cu) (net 10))
 (segment (start 130.81 80.131998) (end 130.81 89.027) (width 0.5) (layer B.Cu) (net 10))
 (segment (start 131.498862 89.715862) (end 132.153138 89.715862) (width 0.5) (layer B.Cu) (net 10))
 (segment (start 130.81 89.027) (end 131.498862 89.715862) (width 0.5) (layer B.Cu) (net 10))
 (segment (start 132.153138 89.715862) (end 133.378462 89.715862) (width 0.5) (layer B.Cu) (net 10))
 (via (at 132.153138 89.715862) (size 0.8) (drill 0.4) (layers F.Cu B.Cu) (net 10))
 (segment (start 127.7874 77.0926) (end 126.72 78.16) (width 0.5) (layer F.Cu) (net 6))
 (segment (start 127.7874 75.3488) (end 127.7874 77.0926) (width 0.5) (layer F.Cu) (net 6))
 (via (at 124.73 77.53) (size 0.5) (drill 0.3) (layers F.Cu B.Cu) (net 5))
 (via (at 124.73 78.28) (size 0.5) (drill 0.3) (layers F.Cu B.Cu) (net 5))
 (via (at 124.73 78.95) (size 0.5) (drill 0.3) (layers F.Cu B.Cu) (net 5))
 (segment (start 125.5268 77.3532) (end 124.72 78.16) (width 0.5) (layer F.Cu) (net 5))
 (segment (start 125.5268 75.368) (end 125.5268 77.3532) (width 0.5) (layer F.Cu) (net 5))
 (segment (start 124.477599 74.318799) (end 125.5268 75.368) (width 0.5) (layer F.Cu) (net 5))
 (segment (start 120.961201 74.318799) (end 124.477599 74.318799) (width 0.5) (layer F.Cu) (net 5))
 (segment (start 120.07 75.21) (end 120.961201 74.318799) (width 0.5) (layer F.Cu) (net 5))
 (via (at 126.74972 64.046) (size 0.5) (drill 0.3) (layers F.Cu B.Cu) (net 12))
 (via (at 124.74972 65.046) (size 0.5) (drill 0.3) (layers F.Cu B.Cu) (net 12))
 (via (at 124.74972 63.046) (size 0.5) (drill 0.3) (layers F.Cu B.Cu) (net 12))
 (via (at 125.74972 63.046) (size 0.5) (drill 0.3) (layers F.Cu B.Cu) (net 12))
 (via (at 126.83 63.1) (size 0.5) (drill 0.3) (layers F.Cu B.Cu) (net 12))
 (via (at 124.74972 64.046) (size 0.5) (drill 0.3) (layers F.Cu B.Cu) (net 12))
 (via (at 125.7708 64.0092) (size 0.8) (drill 0.4) (layers F.Cu B.Cu) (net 12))
 (via (at 126.74972 65.046) (size 0.5) (drill 0.3) (layers F.Cu B.Cu) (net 12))
 (via (at 125.74972 65.046) (size 0.5) (drill 0.3) (layers F.Cu B.Cu) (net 12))
 (segment (start 122.35 56.38) (end 128.85 56.38) (width 0.5) (layer F.Cu) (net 12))
 (segment (start 127.040001 62.230001) (end 126.82 62.01) (width 0.5) (layer B.Cu) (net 12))
 (segment (start 130.091999 62.230001) (end 127.040001 62.230001) (width 0.5) (layer B.Cu) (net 12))
 (segment (start 131.632 60.69) (end 130.091999 62.230001) (width 0.5) (layer B.Cu) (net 12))
 (segment (start 126.82 58.41) (end 126.82 62.01) (width 0.5) (layer B.Cu) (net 12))
 (segment (start 128.85 56.38) (end 126.82 58.41) (width 0.5) (layer B.Cu) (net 12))
 (segment (start 119.32 61.911998) (end 121.922998 59.309) (width 0.5) (layer B.Cu) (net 12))
 (segment (start 119.32 64.04) (end 119.32 61.911998) (width 0.5) (layer B.Cu) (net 12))
 (segment (start 124.119 59.309) (end 126.82 62.01) (width 0.5) (layer B.Cu) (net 12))
 (segment (start 121.922998 59.309) (end 124.119 59.309) (width 0.5) (layer B.Cu) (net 12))
 (segment (start 125.7808 63.0492) (end 126.82 62.01) (width 0.5) (layer B.Cu) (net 12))
 (segment (start 125.7808 64.0842) (end 125.7808 63.0492) (width 0.5) (layer B.Cu) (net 12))
 (segment (start 128.98 64.17) (end 126.82 62.01) (width 0.5) (layer B.Cu) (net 12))
 (segment (start 130.98 64.17) (end 128.98 64.17) (width 0.5) (layer B.Cu) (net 12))
 (segment (start 133.135003 65.869999) (end 132.330001 65.869999) (width 0.5) (layer B.Cu) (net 13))
 (segment (start 134.099999 64.905003) (end 133.135003 65.869999) (width 0.5) (layer B.Cu) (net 13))
 (segment (start 134.099999 61.778001) (end 134.099999 64.905003) (width 0.5) (layer B.Cu) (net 13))
 (segment (start 132.330001 65.869999) (end 130.98 67.22) (width 0.5) (layer B.Cu) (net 13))
 (segment (start 135.188 60.69) (end 134.099999 61.778001) (width 0.5) (layer B.Cu) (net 13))
 (segment (start 130.048 76.832) (end 128.72 78.16) (width 0.5) (layer F.Cu) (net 7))
 (segment (start 130.048 75.3488) (end 130.048 76.832) (width 0.5) (layer F.Cu) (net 7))
 (segment (start 132.85 64.25) (end 132.85 64.25) (width 0.5) (layer F.Cu) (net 14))
 (segment (start 130.58501 66.64) (end 132.85 64.37501) (width 0.5) (layer F.Cu) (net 14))
 (via (at 132.85 64.37501) (size 0.8) (drill 0.4) (layers F.Cu B.Cu) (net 14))
 (segment (start 122.9 66.64) (end 130.58501 66.64) (width 0.5) (layer F.Cu) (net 14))
 (via (at 122.7836 78.2066) (size 0.5) (drill 0.3) (layers F.Cu B.Cu) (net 4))
 (segment (start 122.7836 68.2036) (end 122.7836 68.2036) (width 0.5) (layer B.Cu) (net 4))
 (segment (start 122.7836 78.2066) (end 122.7836 68.2036) (width 0.5) (layer B.Cu) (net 4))
 (segment (start 122.7836 68.2036) (end 121.22 66.64) (width 0.5) (layer B.Cu) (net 4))
 (via (at 122.7836 68.2036) (size 0.5) (drill 0.3) (layers F.Cu B.Cu) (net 4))
 (segment (start 123.0376 69.9499) (end 123.1575 69.83) (width 0.5) (layer F.Cu) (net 17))
 (segment (start 123.0376 73.0188) (end 123.0376 69.9499) (width 0.5) (layer F.Cu) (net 17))
 (segment (start 123.0376 75.8424) (end 120.72 78.16) (width 0.5) (layer F.Cu) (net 3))
 (segment (start 123.0376 75.4188) (end 123.0376 75.8424) (width 0.5) (layer F.Cu) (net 3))
 (segment (start 131.41 60.495) (end 131.45 60.535) (width 0.5) (layer F.Cu) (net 18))
 (segment (start 131.41 58.52) (end 131.41 60.495) (width 0.5) (layer F.Cu) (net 18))
 (via (at 121.33 64.13) (size 0.8) (drill 0.4) (layers F.Cu B.Cu) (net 16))
 (segment (start 122.35 63.09) (end 121.31 64.13) (width 0.5) (layer F.Cu) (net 16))
 (segment (start 122.35 60.88) (end 122.35 63.09) (width 0.5) (layer F.Cu) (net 16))
 (segment (start 122.35 60.88) (end 128.85 60.88) (width 0.5) (layer F.Cu) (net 16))
 (segment (start 128.85 58.68) (end 131.41 56.12) (width 0.5) (layer F.Cu) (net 16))
 (segment (start 128.85 60.88) (end 128.85 58.68) (width 0.5) (layer F.Cu) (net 16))
 (segment (start 131.41 56.12) (end 131.41 56.135) (width 0.5) (layer F.Cu) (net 16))
 (via (at 120.21 66.67) (size 0.8) (drill 0.4) (layers F.Cu B.Cu) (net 15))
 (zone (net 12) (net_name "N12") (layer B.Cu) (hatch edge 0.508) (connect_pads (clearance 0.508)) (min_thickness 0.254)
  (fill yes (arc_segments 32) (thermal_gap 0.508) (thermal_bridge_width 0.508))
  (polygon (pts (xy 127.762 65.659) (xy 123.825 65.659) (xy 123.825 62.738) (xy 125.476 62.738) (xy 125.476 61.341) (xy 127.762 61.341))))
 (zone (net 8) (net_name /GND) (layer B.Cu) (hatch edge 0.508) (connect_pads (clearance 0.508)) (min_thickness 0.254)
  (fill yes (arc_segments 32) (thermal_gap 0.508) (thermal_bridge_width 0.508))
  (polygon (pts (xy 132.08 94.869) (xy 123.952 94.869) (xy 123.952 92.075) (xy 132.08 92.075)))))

